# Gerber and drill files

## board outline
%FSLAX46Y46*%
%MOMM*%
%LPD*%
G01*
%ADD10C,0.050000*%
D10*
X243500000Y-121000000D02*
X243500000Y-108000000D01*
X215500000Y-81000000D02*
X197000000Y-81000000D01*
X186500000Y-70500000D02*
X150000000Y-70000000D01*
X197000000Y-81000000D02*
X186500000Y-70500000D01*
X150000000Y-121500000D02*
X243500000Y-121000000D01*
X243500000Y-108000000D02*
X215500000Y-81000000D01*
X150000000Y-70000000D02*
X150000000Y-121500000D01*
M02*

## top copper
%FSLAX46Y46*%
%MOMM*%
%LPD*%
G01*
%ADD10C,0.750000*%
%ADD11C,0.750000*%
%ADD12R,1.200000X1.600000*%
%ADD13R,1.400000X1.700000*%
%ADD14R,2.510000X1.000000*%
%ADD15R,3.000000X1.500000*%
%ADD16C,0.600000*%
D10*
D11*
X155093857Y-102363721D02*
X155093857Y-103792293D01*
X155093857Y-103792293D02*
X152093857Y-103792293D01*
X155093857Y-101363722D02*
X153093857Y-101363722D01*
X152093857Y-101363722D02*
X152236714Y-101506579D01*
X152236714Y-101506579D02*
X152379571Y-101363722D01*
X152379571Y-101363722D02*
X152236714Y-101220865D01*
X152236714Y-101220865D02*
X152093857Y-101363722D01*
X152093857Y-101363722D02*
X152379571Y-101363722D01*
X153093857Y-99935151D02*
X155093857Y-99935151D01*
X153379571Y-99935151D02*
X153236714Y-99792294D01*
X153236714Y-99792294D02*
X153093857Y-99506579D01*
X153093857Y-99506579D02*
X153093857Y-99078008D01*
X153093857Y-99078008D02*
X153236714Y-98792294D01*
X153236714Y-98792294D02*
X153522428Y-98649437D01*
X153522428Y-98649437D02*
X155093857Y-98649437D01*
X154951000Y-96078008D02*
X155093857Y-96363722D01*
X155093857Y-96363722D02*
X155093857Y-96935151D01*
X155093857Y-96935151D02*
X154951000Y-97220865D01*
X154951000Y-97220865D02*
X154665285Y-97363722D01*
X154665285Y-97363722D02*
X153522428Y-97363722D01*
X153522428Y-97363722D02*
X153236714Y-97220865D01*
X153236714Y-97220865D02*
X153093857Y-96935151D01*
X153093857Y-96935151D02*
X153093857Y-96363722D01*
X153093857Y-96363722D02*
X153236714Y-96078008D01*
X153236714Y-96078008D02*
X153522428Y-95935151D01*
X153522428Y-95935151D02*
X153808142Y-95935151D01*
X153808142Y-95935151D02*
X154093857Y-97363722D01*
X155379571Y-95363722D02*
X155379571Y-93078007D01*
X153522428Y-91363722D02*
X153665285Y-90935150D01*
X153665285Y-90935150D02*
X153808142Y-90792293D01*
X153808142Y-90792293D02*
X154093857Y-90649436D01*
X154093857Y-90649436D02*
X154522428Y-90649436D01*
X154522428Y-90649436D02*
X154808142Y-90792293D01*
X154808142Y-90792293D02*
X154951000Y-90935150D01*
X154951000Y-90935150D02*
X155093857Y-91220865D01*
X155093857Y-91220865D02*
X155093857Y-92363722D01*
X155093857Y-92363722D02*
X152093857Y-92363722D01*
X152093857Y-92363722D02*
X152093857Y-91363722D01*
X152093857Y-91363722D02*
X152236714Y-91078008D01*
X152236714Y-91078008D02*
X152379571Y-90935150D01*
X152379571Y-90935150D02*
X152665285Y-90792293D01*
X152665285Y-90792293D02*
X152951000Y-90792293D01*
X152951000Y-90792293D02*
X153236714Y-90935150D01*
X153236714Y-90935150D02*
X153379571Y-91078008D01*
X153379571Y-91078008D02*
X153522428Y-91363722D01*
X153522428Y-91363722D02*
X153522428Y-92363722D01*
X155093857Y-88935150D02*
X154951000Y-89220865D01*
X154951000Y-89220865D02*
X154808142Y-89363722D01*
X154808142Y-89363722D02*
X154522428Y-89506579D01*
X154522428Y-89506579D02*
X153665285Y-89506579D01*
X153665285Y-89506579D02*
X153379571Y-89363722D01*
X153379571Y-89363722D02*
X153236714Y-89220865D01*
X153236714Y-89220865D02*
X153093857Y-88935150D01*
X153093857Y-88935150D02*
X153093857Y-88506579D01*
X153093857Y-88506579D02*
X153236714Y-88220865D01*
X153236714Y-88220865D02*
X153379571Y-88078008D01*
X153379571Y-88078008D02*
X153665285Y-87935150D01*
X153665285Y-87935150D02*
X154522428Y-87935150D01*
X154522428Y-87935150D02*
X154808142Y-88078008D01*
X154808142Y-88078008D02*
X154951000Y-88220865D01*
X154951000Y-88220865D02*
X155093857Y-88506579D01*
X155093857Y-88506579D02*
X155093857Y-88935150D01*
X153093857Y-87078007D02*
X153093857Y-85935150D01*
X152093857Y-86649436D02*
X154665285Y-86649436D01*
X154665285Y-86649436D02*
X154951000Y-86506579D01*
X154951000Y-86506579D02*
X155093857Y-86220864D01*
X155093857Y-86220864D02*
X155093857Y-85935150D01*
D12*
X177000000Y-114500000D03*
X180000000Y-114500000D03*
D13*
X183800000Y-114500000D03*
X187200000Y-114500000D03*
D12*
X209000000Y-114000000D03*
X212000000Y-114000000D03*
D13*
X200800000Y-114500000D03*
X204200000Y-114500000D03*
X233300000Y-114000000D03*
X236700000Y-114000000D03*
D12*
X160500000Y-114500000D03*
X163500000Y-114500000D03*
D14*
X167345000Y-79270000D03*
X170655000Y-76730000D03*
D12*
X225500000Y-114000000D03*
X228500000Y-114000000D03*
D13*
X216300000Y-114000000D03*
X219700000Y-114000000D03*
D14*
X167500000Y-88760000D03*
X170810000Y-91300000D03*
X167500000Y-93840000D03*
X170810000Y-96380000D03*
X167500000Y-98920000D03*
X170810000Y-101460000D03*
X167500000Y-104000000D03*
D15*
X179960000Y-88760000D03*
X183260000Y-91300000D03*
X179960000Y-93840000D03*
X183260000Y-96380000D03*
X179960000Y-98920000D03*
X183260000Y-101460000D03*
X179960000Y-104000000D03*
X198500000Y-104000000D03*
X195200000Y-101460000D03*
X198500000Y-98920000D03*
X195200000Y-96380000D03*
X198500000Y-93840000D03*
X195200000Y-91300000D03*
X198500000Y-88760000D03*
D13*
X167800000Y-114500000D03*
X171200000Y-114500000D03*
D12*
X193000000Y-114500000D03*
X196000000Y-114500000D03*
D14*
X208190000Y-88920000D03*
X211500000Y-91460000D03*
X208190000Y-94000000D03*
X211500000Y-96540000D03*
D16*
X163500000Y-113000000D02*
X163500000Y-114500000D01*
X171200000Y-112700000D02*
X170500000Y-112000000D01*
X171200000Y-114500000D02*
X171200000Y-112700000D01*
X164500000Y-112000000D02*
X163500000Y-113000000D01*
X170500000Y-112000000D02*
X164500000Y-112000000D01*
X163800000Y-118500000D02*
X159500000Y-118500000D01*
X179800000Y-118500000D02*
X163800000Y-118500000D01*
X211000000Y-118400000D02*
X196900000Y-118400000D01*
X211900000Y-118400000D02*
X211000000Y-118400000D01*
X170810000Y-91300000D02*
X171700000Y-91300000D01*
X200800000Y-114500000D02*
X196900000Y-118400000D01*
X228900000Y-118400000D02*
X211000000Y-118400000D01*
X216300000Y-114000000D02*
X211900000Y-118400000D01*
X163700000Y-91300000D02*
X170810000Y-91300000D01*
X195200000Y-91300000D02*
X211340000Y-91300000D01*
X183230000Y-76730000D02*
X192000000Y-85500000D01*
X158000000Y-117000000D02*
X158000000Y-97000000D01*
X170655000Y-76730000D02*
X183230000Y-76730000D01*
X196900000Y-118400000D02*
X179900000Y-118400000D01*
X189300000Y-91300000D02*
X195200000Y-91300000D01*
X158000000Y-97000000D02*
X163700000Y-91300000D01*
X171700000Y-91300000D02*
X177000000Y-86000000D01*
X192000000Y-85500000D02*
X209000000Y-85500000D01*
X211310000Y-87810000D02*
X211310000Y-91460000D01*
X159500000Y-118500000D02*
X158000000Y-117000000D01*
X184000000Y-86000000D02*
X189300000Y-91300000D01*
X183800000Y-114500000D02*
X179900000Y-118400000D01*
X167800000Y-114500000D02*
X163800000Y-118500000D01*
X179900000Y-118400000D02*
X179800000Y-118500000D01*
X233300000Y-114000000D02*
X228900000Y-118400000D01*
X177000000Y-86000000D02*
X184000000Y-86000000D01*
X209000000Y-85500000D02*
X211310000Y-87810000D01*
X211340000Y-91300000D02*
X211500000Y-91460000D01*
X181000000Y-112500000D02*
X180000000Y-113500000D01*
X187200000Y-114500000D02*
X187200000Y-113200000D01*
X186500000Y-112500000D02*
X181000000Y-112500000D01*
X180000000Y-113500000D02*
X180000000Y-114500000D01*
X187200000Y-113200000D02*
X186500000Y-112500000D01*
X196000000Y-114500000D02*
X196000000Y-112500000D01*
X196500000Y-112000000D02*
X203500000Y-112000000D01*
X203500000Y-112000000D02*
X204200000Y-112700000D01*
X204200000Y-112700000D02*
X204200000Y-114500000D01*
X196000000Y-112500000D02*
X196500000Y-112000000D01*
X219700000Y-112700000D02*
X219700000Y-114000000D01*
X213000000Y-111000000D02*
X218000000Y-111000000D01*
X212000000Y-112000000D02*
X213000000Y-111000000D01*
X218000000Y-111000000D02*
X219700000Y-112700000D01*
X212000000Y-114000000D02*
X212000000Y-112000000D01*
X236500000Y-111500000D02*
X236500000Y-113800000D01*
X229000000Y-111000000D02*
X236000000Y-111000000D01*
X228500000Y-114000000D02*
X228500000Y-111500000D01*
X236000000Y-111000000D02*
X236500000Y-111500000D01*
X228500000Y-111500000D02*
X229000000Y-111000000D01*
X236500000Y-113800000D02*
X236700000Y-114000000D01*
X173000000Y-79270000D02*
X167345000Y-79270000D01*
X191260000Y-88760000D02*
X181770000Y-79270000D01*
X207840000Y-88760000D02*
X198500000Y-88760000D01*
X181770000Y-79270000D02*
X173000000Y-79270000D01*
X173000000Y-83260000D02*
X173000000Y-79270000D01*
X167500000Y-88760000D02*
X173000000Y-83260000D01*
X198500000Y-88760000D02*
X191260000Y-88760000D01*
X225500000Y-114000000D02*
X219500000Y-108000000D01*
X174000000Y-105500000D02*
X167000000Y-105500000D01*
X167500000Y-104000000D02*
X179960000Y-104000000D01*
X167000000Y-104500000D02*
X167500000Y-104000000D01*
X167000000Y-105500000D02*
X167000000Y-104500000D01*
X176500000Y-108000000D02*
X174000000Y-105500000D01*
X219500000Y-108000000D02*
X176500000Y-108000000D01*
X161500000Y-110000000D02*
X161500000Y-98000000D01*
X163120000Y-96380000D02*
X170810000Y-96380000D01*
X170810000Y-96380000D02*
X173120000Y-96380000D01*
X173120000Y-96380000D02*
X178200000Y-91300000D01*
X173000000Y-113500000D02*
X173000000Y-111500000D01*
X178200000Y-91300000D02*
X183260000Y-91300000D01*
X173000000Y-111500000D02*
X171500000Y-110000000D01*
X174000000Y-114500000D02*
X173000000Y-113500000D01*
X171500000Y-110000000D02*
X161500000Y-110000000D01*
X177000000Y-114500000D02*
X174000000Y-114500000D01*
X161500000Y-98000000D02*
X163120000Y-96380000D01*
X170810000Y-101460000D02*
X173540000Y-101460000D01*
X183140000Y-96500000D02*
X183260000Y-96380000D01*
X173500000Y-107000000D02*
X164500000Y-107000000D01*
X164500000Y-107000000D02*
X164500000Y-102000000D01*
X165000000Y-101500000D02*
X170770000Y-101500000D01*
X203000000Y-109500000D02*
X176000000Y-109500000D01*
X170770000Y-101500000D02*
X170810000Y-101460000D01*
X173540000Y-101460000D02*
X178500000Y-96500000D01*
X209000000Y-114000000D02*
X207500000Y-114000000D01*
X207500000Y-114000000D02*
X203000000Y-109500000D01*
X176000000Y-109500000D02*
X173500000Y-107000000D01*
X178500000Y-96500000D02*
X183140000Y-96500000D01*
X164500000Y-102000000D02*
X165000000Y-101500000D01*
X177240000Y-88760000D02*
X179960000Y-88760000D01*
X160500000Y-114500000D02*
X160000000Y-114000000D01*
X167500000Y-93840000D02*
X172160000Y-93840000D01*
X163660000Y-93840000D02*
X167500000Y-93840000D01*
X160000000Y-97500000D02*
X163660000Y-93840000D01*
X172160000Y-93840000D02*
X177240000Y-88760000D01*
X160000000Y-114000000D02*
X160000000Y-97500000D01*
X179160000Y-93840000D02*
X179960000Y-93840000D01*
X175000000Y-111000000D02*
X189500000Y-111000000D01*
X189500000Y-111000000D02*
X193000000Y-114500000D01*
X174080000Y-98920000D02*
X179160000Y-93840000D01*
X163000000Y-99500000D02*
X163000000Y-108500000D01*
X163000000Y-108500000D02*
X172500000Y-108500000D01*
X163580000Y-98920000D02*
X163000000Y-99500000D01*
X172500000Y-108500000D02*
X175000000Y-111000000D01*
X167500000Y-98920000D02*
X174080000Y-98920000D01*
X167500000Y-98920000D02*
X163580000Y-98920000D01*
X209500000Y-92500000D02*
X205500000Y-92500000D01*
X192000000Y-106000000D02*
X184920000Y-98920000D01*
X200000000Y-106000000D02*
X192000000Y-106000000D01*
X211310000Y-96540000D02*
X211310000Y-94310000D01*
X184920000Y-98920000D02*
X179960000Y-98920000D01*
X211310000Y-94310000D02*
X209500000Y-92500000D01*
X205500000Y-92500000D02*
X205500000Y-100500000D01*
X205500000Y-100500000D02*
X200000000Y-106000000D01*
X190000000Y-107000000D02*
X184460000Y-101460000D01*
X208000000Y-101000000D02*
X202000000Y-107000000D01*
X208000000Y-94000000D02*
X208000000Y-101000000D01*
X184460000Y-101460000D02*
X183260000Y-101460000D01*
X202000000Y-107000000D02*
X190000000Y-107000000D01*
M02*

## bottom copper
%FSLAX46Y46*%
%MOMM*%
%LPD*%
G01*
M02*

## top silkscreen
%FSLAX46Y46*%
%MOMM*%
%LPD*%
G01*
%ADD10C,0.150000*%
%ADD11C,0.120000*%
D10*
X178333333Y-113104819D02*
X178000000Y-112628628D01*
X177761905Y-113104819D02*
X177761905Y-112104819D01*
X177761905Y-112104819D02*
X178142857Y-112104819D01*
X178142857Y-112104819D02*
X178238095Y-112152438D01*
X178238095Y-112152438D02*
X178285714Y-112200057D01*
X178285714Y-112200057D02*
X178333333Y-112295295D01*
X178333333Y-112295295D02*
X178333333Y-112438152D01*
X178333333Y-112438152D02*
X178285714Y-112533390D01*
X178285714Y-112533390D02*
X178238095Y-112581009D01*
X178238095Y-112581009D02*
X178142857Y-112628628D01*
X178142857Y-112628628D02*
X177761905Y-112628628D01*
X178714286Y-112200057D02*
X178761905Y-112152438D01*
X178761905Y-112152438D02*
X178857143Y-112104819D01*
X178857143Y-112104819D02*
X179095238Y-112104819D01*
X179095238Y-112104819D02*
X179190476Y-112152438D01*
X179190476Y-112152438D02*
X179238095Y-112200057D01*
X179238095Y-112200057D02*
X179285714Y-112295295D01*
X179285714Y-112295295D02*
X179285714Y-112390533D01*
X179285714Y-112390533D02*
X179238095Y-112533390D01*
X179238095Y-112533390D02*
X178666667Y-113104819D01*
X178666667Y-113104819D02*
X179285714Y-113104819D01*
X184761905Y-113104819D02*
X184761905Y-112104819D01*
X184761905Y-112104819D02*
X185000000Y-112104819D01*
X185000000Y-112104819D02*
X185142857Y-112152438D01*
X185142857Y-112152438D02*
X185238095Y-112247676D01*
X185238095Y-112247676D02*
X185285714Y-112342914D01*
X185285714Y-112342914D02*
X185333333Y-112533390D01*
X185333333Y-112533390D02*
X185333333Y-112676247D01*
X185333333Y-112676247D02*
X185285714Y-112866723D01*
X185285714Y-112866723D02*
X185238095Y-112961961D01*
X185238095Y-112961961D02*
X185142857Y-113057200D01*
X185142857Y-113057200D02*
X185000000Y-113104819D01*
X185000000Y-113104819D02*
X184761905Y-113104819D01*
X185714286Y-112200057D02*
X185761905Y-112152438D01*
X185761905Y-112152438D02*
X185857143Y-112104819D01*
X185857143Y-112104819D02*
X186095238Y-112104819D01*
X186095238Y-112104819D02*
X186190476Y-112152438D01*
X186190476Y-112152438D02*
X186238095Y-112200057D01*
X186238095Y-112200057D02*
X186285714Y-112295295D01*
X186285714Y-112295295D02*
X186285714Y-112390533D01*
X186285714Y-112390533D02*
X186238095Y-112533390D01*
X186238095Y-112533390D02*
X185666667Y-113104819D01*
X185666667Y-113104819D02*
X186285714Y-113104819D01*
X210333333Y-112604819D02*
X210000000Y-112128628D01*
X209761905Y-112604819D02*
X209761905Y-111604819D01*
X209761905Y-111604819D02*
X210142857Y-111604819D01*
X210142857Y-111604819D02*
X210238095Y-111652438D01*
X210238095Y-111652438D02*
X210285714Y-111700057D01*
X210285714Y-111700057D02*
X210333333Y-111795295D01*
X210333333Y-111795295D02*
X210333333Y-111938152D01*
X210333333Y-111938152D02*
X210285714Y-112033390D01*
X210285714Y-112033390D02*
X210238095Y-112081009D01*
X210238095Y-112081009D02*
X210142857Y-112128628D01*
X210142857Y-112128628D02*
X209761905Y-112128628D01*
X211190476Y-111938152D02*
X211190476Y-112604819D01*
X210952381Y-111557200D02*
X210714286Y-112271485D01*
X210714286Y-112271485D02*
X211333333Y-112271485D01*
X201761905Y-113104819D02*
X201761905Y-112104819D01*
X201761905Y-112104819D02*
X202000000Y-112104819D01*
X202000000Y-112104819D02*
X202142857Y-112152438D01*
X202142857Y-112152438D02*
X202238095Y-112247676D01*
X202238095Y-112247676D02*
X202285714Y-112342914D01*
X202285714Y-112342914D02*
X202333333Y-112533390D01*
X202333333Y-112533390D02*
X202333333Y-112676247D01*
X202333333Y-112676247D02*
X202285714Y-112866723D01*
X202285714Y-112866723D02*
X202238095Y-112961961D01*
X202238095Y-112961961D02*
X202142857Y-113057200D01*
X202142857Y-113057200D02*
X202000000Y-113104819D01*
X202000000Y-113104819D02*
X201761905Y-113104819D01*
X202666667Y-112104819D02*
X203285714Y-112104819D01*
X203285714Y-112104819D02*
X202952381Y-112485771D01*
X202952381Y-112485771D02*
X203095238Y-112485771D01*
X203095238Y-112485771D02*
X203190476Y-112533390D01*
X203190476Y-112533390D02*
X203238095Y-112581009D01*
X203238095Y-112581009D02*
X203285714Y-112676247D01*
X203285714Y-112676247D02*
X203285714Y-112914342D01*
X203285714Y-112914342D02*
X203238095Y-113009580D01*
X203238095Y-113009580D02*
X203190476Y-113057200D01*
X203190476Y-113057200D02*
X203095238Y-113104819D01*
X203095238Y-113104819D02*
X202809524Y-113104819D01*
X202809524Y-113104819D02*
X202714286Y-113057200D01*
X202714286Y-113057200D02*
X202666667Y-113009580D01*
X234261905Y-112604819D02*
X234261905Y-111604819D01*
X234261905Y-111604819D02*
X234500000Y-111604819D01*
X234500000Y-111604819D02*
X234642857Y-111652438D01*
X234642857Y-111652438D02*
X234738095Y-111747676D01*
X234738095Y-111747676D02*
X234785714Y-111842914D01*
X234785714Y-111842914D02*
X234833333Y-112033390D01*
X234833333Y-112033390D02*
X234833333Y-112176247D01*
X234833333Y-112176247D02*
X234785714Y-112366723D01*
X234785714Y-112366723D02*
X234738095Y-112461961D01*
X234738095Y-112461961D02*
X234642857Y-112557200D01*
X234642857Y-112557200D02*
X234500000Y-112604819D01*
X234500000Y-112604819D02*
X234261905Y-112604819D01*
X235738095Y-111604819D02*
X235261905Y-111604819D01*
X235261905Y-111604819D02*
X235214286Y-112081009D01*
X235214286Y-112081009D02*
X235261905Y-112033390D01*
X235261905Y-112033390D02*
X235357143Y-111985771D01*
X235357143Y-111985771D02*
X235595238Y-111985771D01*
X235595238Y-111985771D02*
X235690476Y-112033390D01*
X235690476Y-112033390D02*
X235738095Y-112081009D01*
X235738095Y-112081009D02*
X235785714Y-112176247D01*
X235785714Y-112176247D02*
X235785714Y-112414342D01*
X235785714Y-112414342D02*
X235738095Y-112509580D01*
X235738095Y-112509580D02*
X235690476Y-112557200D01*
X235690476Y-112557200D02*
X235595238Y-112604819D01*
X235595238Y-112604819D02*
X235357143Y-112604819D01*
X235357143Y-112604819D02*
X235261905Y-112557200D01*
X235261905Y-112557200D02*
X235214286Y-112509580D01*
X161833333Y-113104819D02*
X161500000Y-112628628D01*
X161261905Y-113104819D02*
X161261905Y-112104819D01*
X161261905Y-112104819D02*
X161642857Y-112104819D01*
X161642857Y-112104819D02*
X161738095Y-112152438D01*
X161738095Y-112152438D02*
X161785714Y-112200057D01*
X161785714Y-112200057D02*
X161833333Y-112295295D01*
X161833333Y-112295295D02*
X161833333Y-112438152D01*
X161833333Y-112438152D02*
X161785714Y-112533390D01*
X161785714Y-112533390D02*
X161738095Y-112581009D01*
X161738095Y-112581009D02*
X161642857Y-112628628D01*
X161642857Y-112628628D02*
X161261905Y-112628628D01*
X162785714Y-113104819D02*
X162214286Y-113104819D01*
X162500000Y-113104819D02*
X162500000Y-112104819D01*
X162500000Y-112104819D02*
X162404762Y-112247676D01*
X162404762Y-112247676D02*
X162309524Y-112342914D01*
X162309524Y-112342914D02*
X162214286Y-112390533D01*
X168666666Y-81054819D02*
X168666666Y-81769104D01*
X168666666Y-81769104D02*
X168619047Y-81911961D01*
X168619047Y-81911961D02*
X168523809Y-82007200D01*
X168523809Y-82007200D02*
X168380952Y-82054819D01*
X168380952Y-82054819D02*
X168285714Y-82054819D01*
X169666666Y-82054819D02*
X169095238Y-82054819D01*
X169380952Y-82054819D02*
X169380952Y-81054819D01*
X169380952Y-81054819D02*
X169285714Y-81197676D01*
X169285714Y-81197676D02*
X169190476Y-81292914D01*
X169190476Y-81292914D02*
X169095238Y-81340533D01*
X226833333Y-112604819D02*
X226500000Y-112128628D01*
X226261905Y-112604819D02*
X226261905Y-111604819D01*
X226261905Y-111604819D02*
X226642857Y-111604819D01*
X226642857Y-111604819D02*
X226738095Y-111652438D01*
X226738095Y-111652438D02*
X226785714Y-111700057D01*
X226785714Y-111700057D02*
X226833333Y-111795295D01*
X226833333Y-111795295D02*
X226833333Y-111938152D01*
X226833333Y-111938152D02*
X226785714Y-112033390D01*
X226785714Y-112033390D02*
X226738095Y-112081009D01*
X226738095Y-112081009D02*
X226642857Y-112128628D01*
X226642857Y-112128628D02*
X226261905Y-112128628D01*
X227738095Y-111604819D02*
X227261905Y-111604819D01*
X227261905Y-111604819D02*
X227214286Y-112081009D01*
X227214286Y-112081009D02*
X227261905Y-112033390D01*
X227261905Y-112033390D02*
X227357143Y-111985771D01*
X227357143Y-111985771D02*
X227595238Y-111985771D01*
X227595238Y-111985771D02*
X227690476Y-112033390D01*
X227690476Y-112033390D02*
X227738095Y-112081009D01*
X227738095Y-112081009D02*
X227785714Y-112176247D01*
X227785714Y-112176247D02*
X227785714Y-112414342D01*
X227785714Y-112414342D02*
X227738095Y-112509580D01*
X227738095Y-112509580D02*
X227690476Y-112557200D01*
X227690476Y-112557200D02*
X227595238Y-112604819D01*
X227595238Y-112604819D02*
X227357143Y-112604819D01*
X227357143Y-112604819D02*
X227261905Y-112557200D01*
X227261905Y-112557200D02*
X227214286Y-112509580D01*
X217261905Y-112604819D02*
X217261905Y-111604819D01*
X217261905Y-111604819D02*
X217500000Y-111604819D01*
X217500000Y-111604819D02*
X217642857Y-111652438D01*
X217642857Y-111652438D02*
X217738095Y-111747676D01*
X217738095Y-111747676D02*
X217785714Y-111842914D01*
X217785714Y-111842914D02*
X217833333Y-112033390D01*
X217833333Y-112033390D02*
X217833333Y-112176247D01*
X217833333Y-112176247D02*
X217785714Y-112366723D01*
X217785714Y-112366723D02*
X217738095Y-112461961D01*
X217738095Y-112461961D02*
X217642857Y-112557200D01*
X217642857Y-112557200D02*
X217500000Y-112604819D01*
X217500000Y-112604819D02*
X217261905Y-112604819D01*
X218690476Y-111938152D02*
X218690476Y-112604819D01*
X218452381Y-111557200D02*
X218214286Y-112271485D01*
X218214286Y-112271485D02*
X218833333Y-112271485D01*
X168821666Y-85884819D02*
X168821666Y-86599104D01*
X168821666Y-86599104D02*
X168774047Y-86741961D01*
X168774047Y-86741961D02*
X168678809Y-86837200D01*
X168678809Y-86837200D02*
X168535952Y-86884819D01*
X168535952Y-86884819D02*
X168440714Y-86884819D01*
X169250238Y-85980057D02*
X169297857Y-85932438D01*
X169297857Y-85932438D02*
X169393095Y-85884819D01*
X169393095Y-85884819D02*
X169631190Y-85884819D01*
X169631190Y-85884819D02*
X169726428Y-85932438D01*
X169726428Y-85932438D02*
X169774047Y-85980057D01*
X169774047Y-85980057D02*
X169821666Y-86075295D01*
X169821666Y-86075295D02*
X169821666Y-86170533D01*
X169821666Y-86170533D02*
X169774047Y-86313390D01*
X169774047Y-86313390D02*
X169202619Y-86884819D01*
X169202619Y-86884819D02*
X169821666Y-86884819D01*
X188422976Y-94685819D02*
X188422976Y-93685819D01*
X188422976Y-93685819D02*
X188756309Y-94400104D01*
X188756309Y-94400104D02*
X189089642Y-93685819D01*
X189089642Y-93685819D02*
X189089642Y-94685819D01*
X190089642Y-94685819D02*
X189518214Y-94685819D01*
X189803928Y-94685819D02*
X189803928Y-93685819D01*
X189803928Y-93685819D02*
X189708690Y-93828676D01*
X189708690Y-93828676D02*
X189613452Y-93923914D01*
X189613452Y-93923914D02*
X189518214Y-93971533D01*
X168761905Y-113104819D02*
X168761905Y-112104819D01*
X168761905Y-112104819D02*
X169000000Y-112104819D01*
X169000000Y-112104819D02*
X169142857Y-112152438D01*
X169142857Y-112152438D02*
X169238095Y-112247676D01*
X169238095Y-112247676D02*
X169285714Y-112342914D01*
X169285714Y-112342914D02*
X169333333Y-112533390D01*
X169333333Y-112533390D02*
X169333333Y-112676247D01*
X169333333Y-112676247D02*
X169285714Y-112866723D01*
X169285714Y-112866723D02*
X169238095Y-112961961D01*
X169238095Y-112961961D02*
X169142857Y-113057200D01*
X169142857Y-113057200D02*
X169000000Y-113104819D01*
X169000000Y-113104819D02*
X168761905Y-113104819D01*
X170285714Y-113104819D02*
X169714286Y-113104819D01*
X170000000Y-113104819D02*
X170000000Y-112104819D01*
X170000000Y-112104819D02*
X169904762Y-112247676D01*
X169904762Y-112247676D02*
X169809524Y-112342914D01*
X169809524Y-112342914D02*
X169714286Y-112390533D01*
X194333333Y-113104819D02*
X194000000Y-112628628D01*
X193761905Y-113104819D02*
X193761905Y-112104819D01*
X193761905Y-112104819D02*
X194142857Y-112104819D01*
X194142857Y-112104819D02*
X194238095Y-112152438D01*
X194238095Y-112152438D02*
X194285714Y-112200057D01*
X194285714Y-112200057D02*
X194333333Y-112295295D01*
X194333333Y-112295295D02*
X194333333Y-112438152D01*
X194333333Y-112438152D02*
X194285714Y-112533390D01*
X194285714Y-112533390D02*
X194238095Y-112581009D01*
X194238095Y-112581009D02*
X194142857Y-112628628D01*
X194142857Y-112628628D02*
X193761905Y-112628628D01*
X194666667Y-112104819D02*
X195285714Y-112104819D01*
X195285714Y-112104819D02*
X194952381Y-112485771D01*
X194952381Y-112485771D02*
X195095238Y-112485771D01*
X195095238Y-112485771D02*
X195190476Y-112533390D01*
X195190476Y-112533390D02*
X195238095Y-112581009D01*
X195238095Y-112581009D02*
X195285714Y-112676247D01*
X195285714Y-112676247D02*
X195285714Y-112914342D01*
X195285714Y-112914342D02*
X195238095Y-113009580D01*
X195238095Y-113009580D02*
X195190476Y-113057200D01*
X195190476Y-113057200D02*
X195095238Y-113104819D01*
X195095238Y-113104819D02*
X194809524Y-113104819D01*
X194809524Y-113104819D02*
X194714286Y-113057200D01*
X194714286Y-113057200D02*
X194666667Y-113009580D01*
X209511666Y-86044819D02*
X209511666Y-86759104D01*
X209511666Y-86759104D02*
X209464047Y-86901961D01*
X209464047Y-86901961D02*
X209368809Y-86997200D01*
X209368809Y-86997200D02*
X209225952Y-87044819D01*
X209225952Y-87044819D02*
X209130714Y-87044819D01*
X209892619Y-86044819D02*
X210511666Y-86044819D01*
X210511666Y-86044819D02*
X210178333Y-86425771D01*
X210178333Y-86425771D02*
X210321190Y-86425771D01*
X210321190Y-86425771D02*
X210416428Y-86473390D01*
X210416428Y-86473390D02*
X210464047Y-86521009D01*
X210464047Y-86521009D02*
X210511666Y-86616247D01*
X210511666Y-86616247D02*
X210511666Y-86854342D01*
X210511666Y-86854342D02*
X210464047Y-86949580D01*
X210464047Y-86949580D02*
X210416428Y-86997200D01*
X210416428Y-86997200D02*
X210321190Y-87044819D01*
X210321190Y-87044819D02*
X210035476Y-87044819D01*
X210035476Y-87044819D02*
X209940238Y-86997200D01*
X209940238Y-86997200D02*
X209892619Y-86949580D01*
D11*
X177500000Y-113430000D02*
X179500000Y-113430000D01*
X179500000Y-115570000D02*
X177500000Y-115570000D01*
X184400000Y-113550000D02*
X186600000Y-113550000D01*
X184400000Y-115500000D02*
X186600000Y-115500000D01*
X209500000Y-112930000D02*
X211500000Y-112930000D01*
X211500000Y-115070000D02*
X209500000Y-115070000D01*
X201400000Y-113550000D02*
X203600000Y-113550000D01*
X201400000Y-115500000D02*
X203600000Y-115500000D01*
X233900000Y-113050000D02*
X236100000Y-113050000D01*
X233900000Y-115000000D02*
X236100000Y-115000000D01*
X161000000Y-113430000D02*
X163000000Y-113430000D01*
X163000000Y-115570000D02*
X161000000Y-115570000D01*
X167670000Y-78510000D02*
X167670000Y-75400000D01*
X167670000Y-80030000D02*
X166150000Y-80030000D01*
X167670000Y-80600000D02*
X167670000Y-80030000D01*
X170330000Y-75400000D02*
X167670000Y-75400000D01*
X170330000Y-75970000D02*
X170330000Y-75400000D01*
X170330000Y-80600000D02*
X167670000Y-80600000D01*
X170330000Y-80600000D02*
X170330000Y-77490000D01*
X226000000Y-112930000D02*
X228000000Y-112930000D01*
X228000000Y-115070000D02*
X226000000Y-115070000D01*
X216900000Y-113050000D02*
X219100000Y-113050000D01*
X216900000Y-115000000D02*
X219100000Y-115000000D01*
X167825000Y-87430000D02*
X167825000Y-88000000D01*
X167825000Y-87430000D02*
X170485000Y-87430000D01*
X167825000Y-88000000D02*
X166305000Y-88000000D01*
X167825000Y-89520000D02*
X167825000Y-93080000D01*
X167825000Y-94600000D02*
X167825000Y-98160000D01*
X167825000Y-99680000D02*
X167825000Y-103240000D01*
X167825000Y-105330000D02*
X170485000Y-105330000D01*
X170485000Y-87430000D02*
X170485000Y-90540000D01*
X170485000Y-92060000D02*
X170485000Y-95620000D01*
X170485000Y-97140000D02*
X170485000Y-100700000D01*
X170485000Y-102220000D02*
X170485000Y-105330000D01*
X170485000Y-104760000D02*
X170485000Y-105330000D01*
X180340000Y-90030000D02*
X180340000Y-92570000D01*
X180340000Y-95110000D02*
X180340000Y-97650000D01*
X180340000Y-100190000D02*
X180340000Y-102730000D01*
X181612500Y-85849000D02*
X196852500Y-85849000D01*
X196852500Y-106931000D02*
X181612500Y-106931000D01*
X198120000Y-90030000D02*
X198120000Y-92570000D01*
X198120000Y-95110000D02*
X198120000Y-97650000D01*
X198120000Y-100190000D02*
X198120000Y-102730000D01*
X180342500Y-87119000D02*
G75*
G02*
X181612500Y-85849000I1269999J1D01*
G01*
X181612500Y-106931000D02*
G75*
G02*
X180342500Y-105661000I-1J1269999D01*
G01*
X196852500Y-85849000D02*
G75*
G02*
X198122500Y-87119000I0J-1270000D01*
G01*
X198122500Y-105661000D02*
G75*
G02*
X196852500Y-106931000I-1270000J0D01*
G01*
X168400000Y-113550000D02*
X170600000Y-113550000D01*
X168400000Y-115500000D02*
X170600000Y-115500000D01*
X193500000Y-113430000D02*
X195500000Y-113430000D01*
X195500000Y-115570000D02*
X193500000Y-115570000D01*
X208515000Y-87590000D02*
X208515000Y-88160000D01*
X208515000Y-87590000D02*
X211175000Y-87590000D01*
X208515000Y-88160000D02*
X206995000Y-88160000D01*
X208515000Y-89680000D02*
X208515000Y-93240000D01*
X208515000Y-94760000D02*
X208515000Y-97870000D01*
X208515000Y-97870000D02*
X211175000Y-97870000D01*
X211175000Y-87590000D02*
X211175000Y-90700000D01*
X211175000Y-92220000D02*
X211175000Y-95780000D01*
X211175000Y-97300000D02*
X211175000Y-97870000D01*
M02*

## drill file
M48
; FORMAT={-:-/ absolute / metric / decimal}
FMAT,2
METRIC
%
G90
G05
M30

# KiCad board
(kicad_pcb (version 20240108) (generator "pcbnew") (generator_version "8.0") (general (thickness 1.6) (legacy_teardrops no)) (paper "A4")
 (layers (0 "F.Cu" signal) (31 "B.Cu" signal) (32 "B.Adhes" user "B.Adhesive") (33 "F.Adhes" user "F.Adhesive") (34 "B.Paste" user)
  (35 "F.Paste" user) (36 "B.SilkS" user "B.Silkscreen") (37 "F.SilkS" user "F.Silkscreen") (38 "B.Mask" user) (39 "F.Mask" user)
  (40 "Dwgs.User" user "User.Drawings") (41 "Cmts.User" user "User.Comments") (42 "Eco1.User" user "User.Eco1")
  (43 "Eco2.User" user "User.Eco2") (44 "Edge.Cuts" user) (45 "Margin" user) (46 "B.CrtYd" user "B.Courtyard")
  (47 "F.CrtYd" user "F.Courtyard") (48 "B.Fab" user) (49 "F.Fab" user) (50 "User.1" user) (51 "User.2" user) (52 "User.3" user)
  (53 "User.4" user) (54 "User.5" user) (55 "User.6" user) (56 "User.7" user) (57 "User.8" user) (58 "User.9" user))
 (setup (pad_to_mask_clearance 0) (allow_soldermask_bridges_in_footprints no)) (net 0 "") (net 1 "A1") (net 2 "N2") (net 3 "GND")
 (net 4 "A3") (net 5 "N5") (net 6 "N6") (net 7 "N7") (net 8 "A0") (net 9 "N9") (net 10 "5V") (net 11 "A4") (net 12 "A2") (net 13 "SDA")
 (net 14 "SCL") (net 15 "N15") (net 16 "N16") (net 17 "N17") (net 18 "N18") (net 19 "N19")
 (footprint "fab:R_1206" (layer "F.Cu") (at 178.5 114.5)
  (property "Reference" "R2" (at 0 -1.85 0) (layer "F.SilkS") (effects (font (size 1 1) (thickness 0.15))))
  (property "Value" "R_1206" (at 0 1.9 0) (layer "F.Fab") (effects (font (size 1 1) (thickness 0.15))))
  (fp_line (start -1 -1.07) (end 1 -1.07) (stroke (width 0.12) (type solid)) (layer "F.SilkS"))
  (fp_line (start 1 1.07) (end -1 1.07) (stroke (width 0.12) (type solid)) (layer "F.SilkS"))
  (pad "1" smd rect (at -1.5 0) (size 1.2 1.6) (layers "F.Cu" "F.Paste" "F.Mask") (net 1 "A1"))
  (pad "2" smd rect (at 1.5 0) (size 1.2 1.6) (layers "F.Cu" "F.Paste" "F.Mask") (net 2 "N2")))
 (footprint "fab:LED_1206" (layer "F.Cu") (at 185.5 114.5)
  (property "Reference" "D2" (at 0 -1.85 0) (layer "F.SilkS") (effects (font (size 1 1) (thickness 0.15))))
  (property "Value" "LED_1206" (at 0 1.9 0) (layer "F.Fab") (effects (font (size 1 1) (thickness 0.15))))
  (fp_line (start -1.1 -0.95) (end 1.1 -0.95) (stroke (width 0.12) (type solid)) (layer "F.SilkS"))
  (fp_line (start -1.1 1) (end 1.1 1) (stroke (width 0.12) (type solid)) (layer "F.SilkS"))
  (pad "1" smd rect (at -1.7 0) (size 1.4 1.7) (layers "F.Cu" "F.Paste" "F.Mask") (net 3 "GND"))
  (pad "2" smd rect (at 1.7 0) (size 1.4 1.7) (layers "F.Cu" "F.Paste" "F.Mask") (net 2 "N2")))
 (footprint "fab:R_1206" (layer "F.Cu") (at 210.5 114)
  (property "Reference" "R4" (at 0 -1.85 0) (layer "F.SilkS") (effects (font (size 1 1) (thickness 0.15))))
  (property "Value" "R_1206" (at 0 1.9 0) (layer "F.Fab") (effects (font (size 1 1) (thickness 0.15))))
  (fp_line (start -1 -1.07) (end 1 -1.07) (stroke (width 0.12) (type solid)) (layer "F.SilkS"))
  (fp_line (start 1 1.07) (end -1 1.07) (stroke (width 0.12) (type solid)) (layer "F.SilkS"))
  (pad "1" smd rect (at -1.5 0) (size 1.2 1.6) (layers "F.Cu" "F.Paste" "F.Mask") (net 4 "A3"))
  (pad "2" smd rect (at 1.5 0) (size 1.2 1.6) (layers "F.Cu" "F.Paste" "F.Mask") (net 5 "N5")))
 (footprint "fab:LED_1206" (layer "F.Cu") (at 202.5 114.5)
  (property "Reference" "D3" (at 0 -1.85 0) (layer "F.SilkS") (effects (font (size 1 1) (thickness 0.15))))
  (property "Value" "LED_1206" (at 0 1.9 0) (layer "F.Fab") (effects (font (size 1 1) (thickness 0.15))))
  (fp_line (start -1.1 -0.95) (end 1.1 -0.95) (stroke (width 0.12) (type solid)) (layer "F.SilkS"))
  (fp_line (start -1.1 1) (end 1.1 1) (stroke (width 0.12) (type solid)) (layer "F.SilkS"))
  (pad "1" smd rect (at -1.7 0) (size 1.4 1.7) (layers "F.Cu" "F.Paste" "F.Mask") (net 3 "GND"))
  (pad "2" smd rect (at 1.7 0) (size 1.4 1.7) (layers "F.Cu" "F.Paste" "F.Mask") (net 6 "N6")))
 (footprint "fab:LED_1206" (layer "F.Cu") (at 235 114)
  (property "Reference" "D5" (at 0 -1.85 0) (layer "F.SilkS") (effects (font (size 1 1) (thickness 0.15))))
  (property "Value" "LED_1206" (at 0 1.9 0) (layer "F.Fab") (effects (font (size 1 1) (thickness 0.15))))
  (fp_line (start -1.1 -0.95) (end 1.1 -0.95) (stroke (width 0.12) (type solid)) (layer "F.SilkS"))
  (fp_line (start -1.1 1) (end 1.1 1) (stroke (width 0.12) (type solid)) (layer "F.SilkS"))
  (pad "1" smd rect (at -1.7 0) (size 1.4 1.7) (layers "F.Cu" "F.Paste" "F.Mask") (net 3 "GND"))
  (pad "2" smd rect (at 1.7 0) (size 1.4 1.7) (layers "F.Cu" "F.Paste" "F.Mask") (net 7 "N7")))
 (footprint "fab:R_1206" (layer "F.Cu") (at 162 114.5)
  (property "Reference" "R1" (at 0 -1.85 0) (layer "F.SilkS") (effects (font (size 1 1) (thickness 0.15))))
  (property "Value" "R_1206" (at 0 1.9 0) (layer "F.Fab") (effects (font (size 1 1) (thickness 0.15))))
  (fp_line (start -1 -1.07) (end 1 -1.07) (stroke (width 0.12) (type solid)) (layer "F.SilkS"))
  (fp_line (start 1 1.07) (end -1 1.07) (stroke (width 0.12) (type solid)) (layer "F.SilkS"))
  (pad "1" smd rect (at -1.5 0) (size 1.2 1.6) (layers "F.Cu" "F.Paste" "F.Mask") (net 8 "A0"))
  (pad "2" smd rect (at 1.5 0) (size 1.2 1.6) (layers "F.Cu" "F.Paste" "F.Mask") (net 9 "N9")))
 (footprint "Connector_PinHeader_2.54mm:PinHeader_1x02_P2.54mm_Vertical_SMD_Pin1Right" (layer "F.Cu") (at 169 78 180)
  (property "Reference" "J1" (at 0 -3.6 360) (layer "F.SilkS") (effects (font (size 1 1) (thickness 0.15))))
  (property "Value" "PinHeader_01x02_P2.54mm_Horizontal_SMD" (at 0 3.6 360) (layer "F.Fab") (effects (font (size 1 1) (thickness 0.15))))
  (fp_line (start 1.33 -0.51) (end 1.33 2.6) (stroke (width 0.12) (type solid)) (layer "F.SilkS"))
  (fp_line (start 1.33 -2.03) (end 2.85 -2.03) (stroke (width 0.12) (type solid)) (layer "F.SilkS"))
  (fp_line (start 1.33 -2.6) (end 1.33 -2.03) (stroke (width 0.12) (type solid)) (layer "F.SilkS"))
  (fp_line (start -1.33 2.6) (end 1.33 2.6) (stroke (width 0.12) (type solid)) (layer "F.SilkS"))
  (fp_line (start -1.33 2.03) (end -1.33 2.6) (stroke (width 0.12) (type solid)) (layer "F.SilkS"))
  (fp_line (start -1.33 -2.6) (end 1.33 -2.6) (stroke (width 0.12) (type solid)) (layer "F.SilkS"))
  (fp_line (start -1.33 -2.6) (end -1.33 0.51) (stroke (width 0.12) (type solid)) (layer "F.SilkS"))
  (pad "1" smd rect (at 1.655 -1.27 180) (size 2.51 1) (layers "F.Cu" "F.Paste" "F.Mask") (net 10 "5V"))
  (pad "2" smd rect (at -1.655 1.27 180) (size 2.51 1) (layers "F.Cu" "F.Paste" "F.Mask") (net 3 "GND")))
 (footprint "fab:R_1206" (layer "F.Cu") (at 227 114)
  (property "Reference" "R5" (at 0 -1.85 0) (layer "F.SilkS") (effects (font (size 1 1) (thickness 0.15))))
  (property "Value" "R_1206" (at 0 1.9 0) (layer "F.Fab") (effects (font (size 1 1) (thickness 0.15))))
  (fp_line (start -1 -1.07) (end 1 -1.07) (stroke (width 0.12) (type solid)) (layer "F.SilkS"))
  (fp_line (start 1 1.07) (end -1 1.07) (stroke (width 0.12) (type solid)) (layer "F.SilkS"))
  (pad "1" smd rect (at -1.5 0) (size 1.2 1.6) (layers "F.Cu" "F.Paste" "F.Mask") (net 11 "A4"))
  (pad "2" smd rect (at 1.5 0) (size 1.2 1.6) (layers "F.Cu" "F.Paste" "F.Mask") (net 7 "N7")))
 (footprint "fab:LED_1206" (layer "F.Cu") (at 218 114)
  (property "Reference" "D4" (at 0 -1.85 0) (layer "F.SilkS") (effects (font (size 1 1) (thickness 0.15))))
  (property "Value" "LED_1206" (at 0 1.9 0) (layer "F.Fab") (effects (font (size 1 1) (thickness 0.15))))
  (fp_line (start -1.1 -0.95) (end 1.1 -0.95) (stroke (width 0.12) (type solid)) (layer "F.SilkS"))
  (fp_line (start -1.1 1) (end 1.1 1) (stroke (width 0.12) (type solid)) (layer "F.SilkS"))
  (pad "1" smd rect (at -1.7 0) (size 1.4 1.7) (layers "F.Cu" "F.Paste" "F.Mask") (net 3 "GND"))
  (pad "2" smd rect (at 1.7 0) (size 1.4 1.7) (layers "F.Cu" "F.Paste" "F.Mask") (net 5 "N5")))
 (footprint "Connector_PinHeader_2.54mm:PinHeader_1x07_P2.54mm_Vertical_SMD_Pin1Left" (layer "F.Cu") (at 169.155 96.38)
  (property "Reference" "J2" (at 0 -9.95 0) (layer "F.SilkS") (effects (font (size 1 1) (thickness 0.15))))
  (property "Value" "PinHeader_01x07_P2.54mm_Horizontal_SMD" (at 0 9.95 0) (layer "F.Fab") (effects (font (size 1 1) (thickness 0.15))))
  (fp_line (start -1.33 -8.95) (end -1.33 -8.38) (stroke (width 0.12) (type solid)) (layer "F.SilkS"))
  (fp_line (start -1.33 -8.95) (end 1.33 -8.95) (stroke (width 0.12) (type solid)) (layer "F.SilkS"))
  (fp_line (start -1.33 -8.38) (end -2.85 -8.38) (stroke (width 0.12) (type solid)) (layer "F.SilkS"))
  (fp_line (start -1.33 -6.86) (end -1.33 -3.3) (stroke (width 0.12) (type solid)) (layer "F.SilkS"))
  (fp_line (start -1.33 -1.78) (end -1.33 1.78) (stroke (width 0.12) (type solid)) (layer "F.SilkS"))
  (fp_line (start -1.33 3.3) (end -1.33 6.86) (stroke (width 0.12) (type solid)) (layer "F.SilkS"))
  (fp_line (start -1.33 8.95) (end 1.33 8.95) (stroke (width 0.12) (type solid)) (layer "F.SilkS"))
  (fp_line (start 1.33 -8.95) (end 1.33 -5.84) (stroke (width 0.12) (type solid)) (layer "F.SilkS"))
  (fp_line (start 1.33 -4.32) (end 1.33 -0.76) (stroke (width 0.12) (type solid)) (layer "F.SilkS"))
  (fp_line (start 1.33 0.76) (end 1.33 4.32) (stroke (width 0.12) (type solid)) (layer "F.SilkS"))
  (fp_line (start 1.33 5.84) (end 1.33 8.95) (stroke (width 0.12) (type solid)) (layer "F.SilkS"))
  (fp_line (start 1.33 8.38) (end 1.33 8.95) (stroke (width 0.12) (type solid)) (layer "F.SilkS"))
  (pad "1" smd rect (at -1.655 -7.62) (size 2.51 1) (layers "F.Cu" "F.Paste" "F.Mask") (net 10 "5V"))
  (pad "2" smd rect (at 1.655 -5.08) (size 2.51 1) (layers "F.Cu" "F.Paste" "F.Mask") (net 3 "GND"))
  (pad "3" smd rect (at -1.655 -2.54) (size 2.51 1) (layers "F.Cu" "F.Paste" "F.Mask") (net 8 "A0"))
  (pad "4" smd rect (at 1.655 0) (size 2.51 1) (layers "F.Cu" "F.Paste" "F.Mask") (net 1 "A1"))
  (pad "5" smd rect (at -1.655 2.54) (size 2.51 1) (layers "F.Cu" "F.Paste" "F.Mask") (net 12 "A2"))
  (pad "6" smd rect (at 1.655 5.08) (size 2.51 1) (layers "F.Cu" "F.Paste" "F.Mask") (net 4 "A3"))
  (pad "7" smd rect (at -1.655 7.62) (size 2.51 1) (layers "F.Cu" "F.Paste" "F.Mask") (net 11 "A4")))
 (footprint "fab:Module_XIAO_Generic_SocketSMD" (layer "F.Cu") (at 189.23 96.38)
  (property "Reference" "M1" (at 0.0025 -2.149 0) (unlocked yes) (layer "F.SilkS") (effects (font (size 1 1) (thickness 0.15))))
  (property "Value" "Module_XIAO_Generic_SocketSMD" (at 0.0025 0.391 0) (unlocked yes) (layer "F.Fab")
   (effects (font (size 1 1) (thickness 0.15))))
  (fp_line (start -8.89 -6.35) (end -8.89 -3.81) (stroke (width 0.12) (type default)) (layer "F.SilkS"))
  (fp_line (start -8.89 -1.27) (end -8.89 1.27) (stroke (width 0.12) (type default)) (layer "F.SilkS"))
  (fp_line (start -8.89 3.81) (end -8.89 6.35) (stroke (width 0.12) (type default)) (layer "F.SilkS"))
  (fp_line (start -7.6175 -10.531) (end 7.6225 -10.531) (stroke (width 0.12) (type solid)) (layer "F.SilkS"))
  (fp_line (start 7.6225 10.551) (end -7.6175 10.551) (stroke (width 0.12) (type solid)) (layer "F.SilkS"))
  (fp_line (start 8.89 -6.35) (end 8.89 -3.81) (stroke (width 0.12) (type default)) (layer "F.SilkS"))
  (fp_line (start 8.89 -1.27) (end 8.89 1.27) (stroke (width 0.12) (type default)) (layer "F.SilkS"))
  (fp_line (start 8.89 3.81) (end 8.89 6.35) (stroke (width 0.12) (type default)) (layer "F.SilkS"))
  (fp_arc (start -8.8875 -9.261) (mid -8.515526 -10.159026) (end -7.6175 -10.531) (stroke (width 0.12) (type solid)) (layer "F.SilkS"))
  (fp_arc (start -7.6175 10.551) (mid -8.515526 10.179026) (end -8.8875 9.281) (stroke (width 0.12) (type solid)) (layer "F.SilkS"))
  (fp_arc (start 7.6225 -10.531) (mid 8.520526 -10.159026) (end 8.8925 -9.261) (stroke (width 0.12) (type solid)) (layer "F.SilkS"))
  (fp_arc (start 8.8925 9.281) (mid 8.520526 10.179026) (end 7.6225 10.551) (stroke (width 0.12) (type solid)) (layer "F.SilkS"))
  (pad "1" smd rect (at -9.27 -7.62) (size 3 1.5) (layers "F.Cu" "F.Paste" "F.Mask") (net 8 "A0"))
  (pad "2" smd rect (at -5.97 -5.08) (size 3 1.5) (layers "F.Cu" "F.Paste" "F.Mask") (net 1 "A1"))
  (pad "3" smd rect (at -9.27 -2.54) (size 3 1.5) (layers "F.Cu" "F.Paste" "F.Mask") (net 12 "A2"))
  (pad "4" smd rect (at -5.97 0) (size 3 1.5) (layers "F.Cu" "F.Paste" "F.Mask") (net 4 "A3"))
  (pad "5" smd rect (at -9.27 2.54) (size 3 1.5) (layers "F.Cu" "F.Paste" "F.Mask") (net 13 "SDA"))
  (pad "6" smd rect (at -5.97 5.08) (size 3 1.5) (layers "F.Cu" "F.Paste" "F.Mask") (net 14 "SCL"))
  (pad "7" smd rect (at -9.27 7.62) (size 3 1.5) (layers "F.Cu" "F.Paste" "F.Mask") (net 11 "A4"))
  (pad "8" smd rect (at 9.27 7.62) (size 3 1.5) (layers "F.Cu" "F.Paste" "F.Mask") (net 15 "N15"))
  (pad "9" smd rect (at 5.97 5.08) (size 3 1.5) (layers "F.Cu" "F.Paste" "F.Mask") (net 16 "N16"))
  (pad "10" smd rect (at 9.27 2.54) (size 3 1.5) (layers "F.Cu" "F.Paste" "F.Mask") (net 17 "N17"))
  (pad "11" smd rect (at 5.97 0) (size 3 1.5) (layers "F.Cu" "F.Paste" "F.Mask") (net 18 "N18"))
  (pad "12" smd rect (at 9.27 -2.54) (size 3 1.5) (layers "F.Cu" "F.Paste" "F.Mask") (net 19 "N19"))
  (pad "13" smd rect (at 5.97 -5.08) (size 3 1.5) (layers "F.Cu" "F.Paste" "F.Mask") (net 3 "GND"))
  (pad "14" smd rect (at 9.27 -7.62) (size 3 1.5) (layers "F.Cu" "F.Paste" "F.Mask") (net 10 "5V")))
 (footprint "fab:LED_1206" (layer "F.Cu") (at 169.5 114.5)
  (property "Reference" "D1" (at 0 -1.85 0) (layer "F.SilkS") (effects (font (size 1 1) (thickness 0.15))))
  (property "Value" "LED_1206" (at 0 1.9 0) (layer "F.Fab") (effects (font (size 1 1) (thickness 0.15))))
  (fp_line (start -1.1 -0.95) (end 1.1 -0.95) (stroke (width 0.12) (type solid)) (layer "F.SilkS"))
  (fp_line (start -1.1 1) (end 1.1 1) (stroke (width 0.12) (type solid)) (layer "F.SilkS"))
  (pad "1" smd rect (at -1.7 0) (size 1.4 1.7) (layers "F.Cu" "F.Paste" "F.Mask") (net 3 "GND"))
  (pad "2" smd rect (at 1.7 0) (size 1.4 1.7) (layers "F.Cu" "F.Paste" "F.Mask") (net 9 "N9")))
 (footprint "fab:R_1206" (layer "F.Cu") (at 194.5 114.5)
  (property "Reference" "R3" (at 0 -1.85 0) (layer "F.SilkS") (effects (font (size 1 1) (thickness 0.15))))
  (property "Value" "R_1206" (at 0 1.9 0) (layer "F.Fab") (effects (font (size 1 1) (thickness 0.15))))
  (fp_line (start -1 -1.07) (end 1 -1.07) (stroke (width 0.12) (type solid)) (layer "F.SilkS"))
  (fp_line (start 1 1.07) (end -1 1.07) (stroke (width 0.12) (type solid)) (layer "F.SilkS"))
  (pad "1" smd rect (at -1.5 0) (size 1.2 1.6) (layers "F.Cu" "F.Paste" "F.Mask") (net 12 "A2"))
  (pad "2" smd rect (at 1.5 0) (size 1.2 1.6) (layers "F.Cu" "F.Paste" "F.Mask") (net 6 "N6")))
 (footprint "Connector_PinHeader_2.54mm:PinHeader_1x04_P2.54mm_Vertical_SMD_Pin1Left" (layer "F.Cu") (at 209.845 92.73)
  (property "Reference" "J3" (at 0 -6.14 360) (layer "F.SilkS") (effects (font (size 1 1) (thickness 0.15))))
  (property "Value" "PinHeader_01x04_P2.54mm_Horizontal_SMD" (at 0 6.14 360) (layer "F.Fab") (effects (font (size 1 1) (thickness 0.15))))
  (fp_line (start -1.33 -5.14) (end -1.33 -4.57) (stroke (width 0.12) (type solid)) (layer "F.SilkS"))
  (fp_line (start -1.33 -5.14) (end 1.33 -5.14) (stroke (width 0.12) (type solid)) (layer "F.SilkS"))
  (fp_line (start -1.33 -4.57) (end -2.85 -4.57) (stroke (width 0.12) (type solid)) (layer "F.SilkS"))
  (fp_line (start -1.33 -3.05) (end -1.33 0.51) (stroke (width 0.12) (type solid)) (layer "F.SilkS"))
  (fp_line (start -1.33 2.03) (end -1.33 5.14) (stroke (width 0.12) (type solid)) (layer "F.SilkS"))
  (fp_line (start -1.33 5.14) (end 1.33 5.14) (stroke (width 0.12) (type solid)) (layer "F.SilkS"))
  (fp_line (start 1.33 -5.14) (end 1.33 -2.03) (stroke (width 0.12) (type solid)) (layer "F.SilkS"))
  (fp_line (start 1.33 -0.51) (end 1.33 3.05) (stroke (width 0.12) (type solid)) (layer "F.SilkS"))
  (fp_line (start 1.33 4.57) (end 1.33 5.14) (stroke (width 0.12) (type solid)) (layer "F.SilkS"))
  (pad "1" smd rect (at -1.655 -3.81) (size 2.51 1) (layers "F.Cu" "F.Paste" "F.Mask") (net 10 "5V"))
  (pad "2" smd rect (at 1.655 -1.27) (size 2.51 1) (layers "F.Cu" "F.Paste" "F.Mask") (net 3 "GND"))
  (pad "3" smd rect (at -1.655 1.27) (size 2.51 1) (layers "F.Cu" "F.Paste" "F.Mask") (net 14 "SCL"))
  (pad "4" smd rect (at 1.655 3.81) (size 2.51 1) (layers "F.Cu" "F.Paste" "F.Mask") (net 13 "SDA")))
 (gr_line (start 243.5 121) (end 243.5 108) (stroke (width 0.05) (type default)) (layer "Edge.Cuts"))
 (gr_line (start 215.5 81) (end 197 81) (stroke (width 0.05) (type default)) (layer "Edge.Cuts"))
 (gr_line (start 186.5 70.5) (end 150 70) (stroke (width 0.05) (type default)) (layer "Edge.Cuts"))
 (gr_line (start 197 81) (end 186.5 70.5) (stroke (width 0.05) (type default)) (layer "Edge.Cuts"))
 (gr_line (start 150 121.5) (end 243.5 121) (stroke (width 0.05) (type default)) (layer "Edge.Cuts"))
 (gr_line (start 243.5 108) (end 215.5 81) (stroke (width 0.05) (type default)) (layer "Edge.Cuts"))
 (gr_line (start 150 70) (end 150 121.5) (stroke (width 0.05) (type default)) (layer "Edge.Cuts"))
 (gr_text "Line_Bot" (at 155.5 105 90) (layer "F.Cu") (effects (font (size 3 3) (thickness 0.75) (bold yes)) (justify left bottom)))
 (segment (start 163.5 113) (end 163.5 114.5) (width 0.6) (layer "F.Cu") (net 9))
 (segment (start 171.2 112.7) (end 170.5 112) (width 0.6) (layer "F.Cu") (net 9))
 (segment (start 171.2 114.5) (end 171.2 112.7) (width 0.6) (layer "F.Cu") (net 9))
 (segment (start 164.5 112) (end 163.5 113) (width 0.6) (layer "F.Cu") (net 9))
 (segment (start 170.5 112) (end 164.5 112) (width 0.6) (layer "F.Cu") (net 9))
 (segment (start 163.8 118.5) (end 159.5 118.5) (width 0.6) (layer "F.Cu") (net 3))
 (segment (start 179.8 118.5) (end 163.8 118.5) (width 0.6) (layer "F.Cu") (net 3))
 (segment (start 211 118.4) (end 196.9 118.4) (width 0.6) (layer "F.Cu") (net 3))
 (segment (start 211.9 118.4) (end 211 118.4) (width 0.6) (layer "F.Cu") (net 3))
 (segment (start 170.81 91.3) (end 171.7 91.3) (width 0.6) (layer "F.Cu") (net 3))
 (segment (start 200.8 114.5) (end 196.9 118.4) (width 0.6) (layer "F.Cu") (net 3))
 (segment (start 228.9 118.4) (end 211 118.4) (width 0.6) (layer "F.Cu") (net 3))
 (segment (start 216.3 114) (end 211.9 118.4) (width 0.6) (layer "F.Cu") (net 3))
 (segment (start 163.7 91.3) (end 170.81 91.3) (width 0.6) (layer "F.Cu") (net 3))
 (segment (start 195.2 91.3) (end 211.34 91.3) (width 0.6) (layer "F.Cu") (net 3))
 (segment (start 183.23 76.73) (end 192 85.5) (width 0.6) (layer "F.Cu") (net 3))
 (segment (start 158 117) (end 158 97) (width 0.6) (layer "F.Cu") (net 3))
 (segment (start 170.655 76.73) (end 183.23 76.73) (width 0.6) (layer "F.Cu") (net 3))
 (segment (start 196.9 118.4) (end 179.9 118.4) (width 0.6) (layer "F.Cu") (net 3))
 (segment (start 189.3 91.3) (end 195.2 91.3) (width 0.6) (layer "F.Cu") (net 3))
 (segment (start 158 97) (end 163.7 91.3) (width 0.6) (layer "F.Cu") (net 3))
 (segment (start 171.7 91.3) (end 177 86) (width 0.6) (layer "F.Cu") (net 3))
 (segment (start 192 85.5) (end 209 85.5) (width 0.6) (layer "F.Cu") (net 3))
 (segment (start 211.31 87.81) (end 211.31 91.46) (width 0.6) (layer "F.Cu") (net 3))
 (segment (start 159.5 118.5) (end 158 117) (width 0.6) (layer "F.Cu") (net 3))
 (segment (start 184 86) (end 189.3 91.3) (width 0.6) (layer "F.Cu") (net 3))
 (segment (start 183.8 114.5) (end 179.9 118.4) (width 0.6) (layer "F.Cu") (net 3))
 (segment (start 167.8 114.5) (end 163.8 118.5) (width 0.6) (layer "F.Cu") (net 3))
 (segment (start 179.9 118.4) (end 179.8 118.5) (width 0.6) (layer "F.Cu") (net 3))
 (segment (start 233.3 114) (end 228.9 118.4) (width 0.6) (layer "F.Cu") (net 3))
 (segment (start 177 86) (end 184 86) (width 0.6) (layer "F.Cu") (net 3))
 (segment (start 209 85.5) (end 211.31 87.81) (width 0.6) (layer "F.Cu") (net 3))
 (segment (start 211.34 91.3) (end 211.5 91.46) (width 0.6) (layer "F.Cu") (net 3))
 (segment (start 181 112.5) (end 180 113.5) (width 0.6) (layer "F.Cu") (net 2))
 (segment (start 187.2 114.5) (end 187.2 113.2) (width 0.6) (layer "F.Cu") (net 2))
 (segment (start 186.5 112.5) (end 181 112.5) (width 0.6) (layer "F.Cu") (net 2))
 (segment (start 180 113.5) (end 180 114.5) (width 0.6) (layer "F.Cu") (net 2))
 (segment (start 187.2 113.2) (end 186.5 112.5) (width 0.6) (layer "F.Cu") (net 2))
 (segment (start 196 114.5) (end 196 112.5) (width 0.6) (layer "F.Cu") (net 6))
 (segment (start 196.5 112) (end 203.5 112) (width 0.6) (layer "F.Cu") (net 6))
 (segment (start 203.5 112) (end 204.2 112.7) (width 0.6) (layer "F.Cu") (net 6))
 (segment (start 204.2 112.7) (end 204.2 114.5) (width 0.6) (layer "F.Cu") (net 6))
 (segment (start 196 112.5) (end 196.5 112) (width 0.6) (layer "F.Cu") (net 6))
 (segment (start 219.7 112.7) (end 219.7 114) (width 0.6) (layer "F.Cu") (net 5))
 (segment (start 213 111) (end 218 111) (width 0.6) (layer "F.Cu") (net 5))
 (segment (start 212 112) (end 213 111) (width 0.6) (layer "F.Cu") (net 5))
 (segment (start 218 111) (end 219.7 112.7) (width 0.6) (layer "F.Cu") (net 5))
 (segment (start 212 114) (end 212 112) (width 0.6) (layer "F.Cu") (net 5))
 (segment (start 236.5 111.5) (end 236.5 113.8) (width 0.6) (layer "F.Cu") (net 7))
 (segment (start 229 111) (end 236 111) (width 0.6) (layer "F.Cu") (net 7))
 (segment (start 228.5 114) (end 228.5 111.5) (width 0.6) (layer "F.Cu") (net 7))
 (segment (start 236 111) (end 236.5 111.5) (width 0.6) (layer "F.Cu") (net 7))
 (segment (start 228.5 111.5) (end 229 111) (width 0.6) (layer "F.Cu") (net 7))
 (segment (start 236.5 113.8) (end 236.7 114) (width 0.6) (layer "F.Cu") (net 7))
 (segment (start 173 79.27) (end 167.345 79.27) (width 0.6) (layer "F.Cu") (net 10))
 (segment (start 191.26 88.76) (end 181.77 79.27) (width 0.6) (layer "F.Cu") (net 10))
 (segment (start 207.84 88.76) (end 198.5 88.76) (width 0.6) (layer "F.Cu") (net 10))
 (segment (start 181.77 79.27) (end 173 79.27) (width 0.6) (layer "F.Cu") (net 10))
 (segment (start 173 83.26) (end 173 79.27) (width 0.6) (layer "F.Cu") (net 10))
 (segment (start 167.5 88.76) (end 173 83.26) (width 0.6) (layer "F.Cu") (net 10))
 (segment (start 198.5 88.76) (end 191.26 88.76) (width 0.6) (layer "F.Cu") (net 10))
 (segment (start 225.5 114) (end 219.5 108) (width 0.6) (layer "F.Cu") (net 11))
 (segment (start 174 105.5) (end 167 105.5) (width 0.6) (layer "F.Cu") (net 11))
 (segment (start 167.5 104) (end 179.96 104) (width 0.6) (layer "F.Cu") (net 11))
 (segment (start 167 104.5) (end 167.5 104) (width 0.6) (layer "F.Cu") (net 11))
 (segment (start 167 105.5) (end 167 104.5) (width 0.6) (layer "F.Cu") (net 11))
 (segment (start 176.5 108) (end 174 105.5) (width 0.6) (layer "F.Cu") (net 11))
 (segment (start 219.5 108) (end 176.5 108) (width 0.6) (layer "F.Cu") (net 11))
 (segment (start 161.5 110) (end 161.5 98) (width 0.6) (layer "F.Cu") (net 1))
 (segment (start 163.12 96.38) (end 170.81 96.38) (width 0.6) (layer "F.Cu") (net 1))
 (segment (start 170.81 96.38) (end 173.12 96.38) (width 0.6) (layer "F.Cu") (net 1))
 (segment (start 173.12 96.38) (end 178.2 91.3) (width 0.6) (layer "F.Cu") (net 1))
 (segment (start 173 113.5) (end 173 111.5) (width 0.6) (layer "F.Cu") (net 1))
 (segment (start 178.2 91.3) (end 183.26 91.3) (width 0.6) (layer "F.Cu") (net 1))
 (segment (start 173 111.5) (end 171.5 110) (width 0.6) (layer "F.Cu") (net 1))
 (segment (start 174 114.5) (end 173 113.5) (width 0.6) (layer "F.Cu") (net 1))
 (segment (start 171.5 110) (end 161.5 110) (width 0.6) (layer "F.Cu") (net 1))
 (segment (start 177 114.5) (end 174 114.5) (width 0.6) (layer "F.Cu") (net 1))
 (segment (start 161.5 98) (end 163.12 96.38) (width 0.6) (layer "F.Cu") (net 1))
 (segment (start 170.81 101.46) (end 173.54 101.46) (width 0.6) (layer "F.Cu") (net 4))
 (segment (start 183.14 96.5) (end 183.26 96.38) (width 0.6) (layer "F.Cu") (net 4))
 (segment (start 173.5 107) (end 164.5 107) (width 0.6) (layer "F.Cu") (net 4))
 (segment (start 164.5 107) (end 164.5 102) (width 0.6) (layer "F.Cu") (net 4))
 (segment (start 165 101.5) (end 170.77 101.5) (width 0.6) (layer "F.Cu") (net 4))
 (segment (start 203 109.5) (end 176 109.5) (width 0.6) (layer "F.Cu") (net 4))
 (segment (start 170.77 101.5) (end 170.81 101.46) (width 0.6) (layer "F.Cu") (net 4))
 (segment (start 173.54 101.46) (end 178.5 96.5) (width 0.6) (layer "F.Cu") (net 4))
 (segment (start 209 114) (end 207.5 114) (width 0.6) (layer "F.Cu") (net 4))
 (segment (start 207.5 114) (end 203 109.5) (width 0.6) (layer "F.Cu") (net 4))
 (segment (start 176 109.5) (end 173.5 107) (width 0.6) (layer "F.Cu") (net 4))
 (segment (start 178.5 96.5) (end 183.14 96.5) (width 0.6) (layer "F.Cu") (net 4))
 (segment (start 164.5 102) (end 165 101.5) (width 0.6) (layer "F.Cu") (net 4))
 (segment (start 177.24 88.76) (end 179.96 88.76) (width 0.6) (layer "F.Cu") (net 8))
 (segment (start 160.5 114.5) (end 160 114) (width 0.6) (layer "F.Cu") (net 8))
 (segment (start 167.5 93.84) (end 172.16 93.84) (width 0.6) (layer "F.Cu") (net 8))
 (segment (start 163.66 93.84) (end 167.5 93.84) (width 0.6) (layer "F.Cu") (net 8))
 (segment (start 160 97.5) (end 163.66 93.84) (width 0.6) (layer "F.Cu") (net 8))
 (segment (start 172.16 93.84) (end 177.24 88.76) (width 0.6) (layer "F.Cu") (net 8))
 (segment (start 160 114) (end 160 97.5) (width 0.6) (layer "F.Cu") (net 8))
 (segment (start 179.16 93.84) (end 179.96 93.84) (width 0.6) (layer "F.Cu") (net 12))
 (segment (start 175 111) (end 189.5 111) (width 0.6) (layer "F.Cu") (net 12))
 (segment (start 189.5 111) (end 193 114.5) (width 0.6) (layer "F.Cu") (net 12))
 (segment (start 174.08 98.92) (end 179.16 93.84) (width 0.6) (layer "F.Cu") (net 12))
 (segment (start 163 99.5) (end 163 108.5) (width 0.6) (layer "F.Cu") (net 12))
 (segment (start 163 108.5) (end 172.5 108.5) (width 0.6) (layer "F.Cu") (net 12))
 (segment (start 163.58 98.92) (end 163 99.5) (width 0.6) (layer "F.Cu") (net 12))
 (segment (start 172.5 108.5) (end 175 111) (width 0.6) (layer "F.Cu") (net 12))
 (segment (start 167.5 98.92) (end 174.08 98.92) (width 0.6) (layer "F.Cu") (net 12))
 (segment (start 167.5 98.92) (end 163.58 98.92) (width 0.6) (layer "F.Cu") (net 12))
 (segment (start 209.5 92.5) (end 205.5 92.5) (width 0.6) (layer "F.Cu") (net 13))
 (segment (start 192 106) (end 184.92 98.92) (width 0.6) (layer "F.Cu") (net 13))
 (segment (start 200 106) (end 192 106) (width 0.6) (layer "F.Cu") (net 13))
 (segment (start 211.31 96.54) (end 211.31 94.31) (width 0.6) (layer "F.Cu") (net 13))
 (segment (start 184.92 98.92) (end 179.96 98.92) (width 0.6) (layer "F.Cu") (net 13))
 (segment (start 211.31 94.31) (end 209.5 92.5) (width 0.6) (layer "F.Cu") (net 13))
 (segment (start 205.5 92.5) (end 205.5 100.5) (width 0.6) (layer "F.Cu") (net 13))
 (segment (start 205.5 100.5) (end 200 106) (width 0.6) (layer "F.Cu") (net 13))
 (segment (start 190 107) (end 184.46 101.46) (width 0.6) (layer "F.Cu") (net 14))
 (segment (start 208 101) (end 202 107) (width 0.6) (layer "F.Cu") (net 14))
 (segment (start 208 94) (end 208 101) (width 0.6) (layer "F.Cu") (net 14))
 (segment (start 184.46 101.46) (end 183.26 101.46) (width 0.6) (layer "F.Cu") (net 14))
 (segment (start 202 107) (end 190 107) (width 0.6) (layer "F.Cu") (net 14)))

